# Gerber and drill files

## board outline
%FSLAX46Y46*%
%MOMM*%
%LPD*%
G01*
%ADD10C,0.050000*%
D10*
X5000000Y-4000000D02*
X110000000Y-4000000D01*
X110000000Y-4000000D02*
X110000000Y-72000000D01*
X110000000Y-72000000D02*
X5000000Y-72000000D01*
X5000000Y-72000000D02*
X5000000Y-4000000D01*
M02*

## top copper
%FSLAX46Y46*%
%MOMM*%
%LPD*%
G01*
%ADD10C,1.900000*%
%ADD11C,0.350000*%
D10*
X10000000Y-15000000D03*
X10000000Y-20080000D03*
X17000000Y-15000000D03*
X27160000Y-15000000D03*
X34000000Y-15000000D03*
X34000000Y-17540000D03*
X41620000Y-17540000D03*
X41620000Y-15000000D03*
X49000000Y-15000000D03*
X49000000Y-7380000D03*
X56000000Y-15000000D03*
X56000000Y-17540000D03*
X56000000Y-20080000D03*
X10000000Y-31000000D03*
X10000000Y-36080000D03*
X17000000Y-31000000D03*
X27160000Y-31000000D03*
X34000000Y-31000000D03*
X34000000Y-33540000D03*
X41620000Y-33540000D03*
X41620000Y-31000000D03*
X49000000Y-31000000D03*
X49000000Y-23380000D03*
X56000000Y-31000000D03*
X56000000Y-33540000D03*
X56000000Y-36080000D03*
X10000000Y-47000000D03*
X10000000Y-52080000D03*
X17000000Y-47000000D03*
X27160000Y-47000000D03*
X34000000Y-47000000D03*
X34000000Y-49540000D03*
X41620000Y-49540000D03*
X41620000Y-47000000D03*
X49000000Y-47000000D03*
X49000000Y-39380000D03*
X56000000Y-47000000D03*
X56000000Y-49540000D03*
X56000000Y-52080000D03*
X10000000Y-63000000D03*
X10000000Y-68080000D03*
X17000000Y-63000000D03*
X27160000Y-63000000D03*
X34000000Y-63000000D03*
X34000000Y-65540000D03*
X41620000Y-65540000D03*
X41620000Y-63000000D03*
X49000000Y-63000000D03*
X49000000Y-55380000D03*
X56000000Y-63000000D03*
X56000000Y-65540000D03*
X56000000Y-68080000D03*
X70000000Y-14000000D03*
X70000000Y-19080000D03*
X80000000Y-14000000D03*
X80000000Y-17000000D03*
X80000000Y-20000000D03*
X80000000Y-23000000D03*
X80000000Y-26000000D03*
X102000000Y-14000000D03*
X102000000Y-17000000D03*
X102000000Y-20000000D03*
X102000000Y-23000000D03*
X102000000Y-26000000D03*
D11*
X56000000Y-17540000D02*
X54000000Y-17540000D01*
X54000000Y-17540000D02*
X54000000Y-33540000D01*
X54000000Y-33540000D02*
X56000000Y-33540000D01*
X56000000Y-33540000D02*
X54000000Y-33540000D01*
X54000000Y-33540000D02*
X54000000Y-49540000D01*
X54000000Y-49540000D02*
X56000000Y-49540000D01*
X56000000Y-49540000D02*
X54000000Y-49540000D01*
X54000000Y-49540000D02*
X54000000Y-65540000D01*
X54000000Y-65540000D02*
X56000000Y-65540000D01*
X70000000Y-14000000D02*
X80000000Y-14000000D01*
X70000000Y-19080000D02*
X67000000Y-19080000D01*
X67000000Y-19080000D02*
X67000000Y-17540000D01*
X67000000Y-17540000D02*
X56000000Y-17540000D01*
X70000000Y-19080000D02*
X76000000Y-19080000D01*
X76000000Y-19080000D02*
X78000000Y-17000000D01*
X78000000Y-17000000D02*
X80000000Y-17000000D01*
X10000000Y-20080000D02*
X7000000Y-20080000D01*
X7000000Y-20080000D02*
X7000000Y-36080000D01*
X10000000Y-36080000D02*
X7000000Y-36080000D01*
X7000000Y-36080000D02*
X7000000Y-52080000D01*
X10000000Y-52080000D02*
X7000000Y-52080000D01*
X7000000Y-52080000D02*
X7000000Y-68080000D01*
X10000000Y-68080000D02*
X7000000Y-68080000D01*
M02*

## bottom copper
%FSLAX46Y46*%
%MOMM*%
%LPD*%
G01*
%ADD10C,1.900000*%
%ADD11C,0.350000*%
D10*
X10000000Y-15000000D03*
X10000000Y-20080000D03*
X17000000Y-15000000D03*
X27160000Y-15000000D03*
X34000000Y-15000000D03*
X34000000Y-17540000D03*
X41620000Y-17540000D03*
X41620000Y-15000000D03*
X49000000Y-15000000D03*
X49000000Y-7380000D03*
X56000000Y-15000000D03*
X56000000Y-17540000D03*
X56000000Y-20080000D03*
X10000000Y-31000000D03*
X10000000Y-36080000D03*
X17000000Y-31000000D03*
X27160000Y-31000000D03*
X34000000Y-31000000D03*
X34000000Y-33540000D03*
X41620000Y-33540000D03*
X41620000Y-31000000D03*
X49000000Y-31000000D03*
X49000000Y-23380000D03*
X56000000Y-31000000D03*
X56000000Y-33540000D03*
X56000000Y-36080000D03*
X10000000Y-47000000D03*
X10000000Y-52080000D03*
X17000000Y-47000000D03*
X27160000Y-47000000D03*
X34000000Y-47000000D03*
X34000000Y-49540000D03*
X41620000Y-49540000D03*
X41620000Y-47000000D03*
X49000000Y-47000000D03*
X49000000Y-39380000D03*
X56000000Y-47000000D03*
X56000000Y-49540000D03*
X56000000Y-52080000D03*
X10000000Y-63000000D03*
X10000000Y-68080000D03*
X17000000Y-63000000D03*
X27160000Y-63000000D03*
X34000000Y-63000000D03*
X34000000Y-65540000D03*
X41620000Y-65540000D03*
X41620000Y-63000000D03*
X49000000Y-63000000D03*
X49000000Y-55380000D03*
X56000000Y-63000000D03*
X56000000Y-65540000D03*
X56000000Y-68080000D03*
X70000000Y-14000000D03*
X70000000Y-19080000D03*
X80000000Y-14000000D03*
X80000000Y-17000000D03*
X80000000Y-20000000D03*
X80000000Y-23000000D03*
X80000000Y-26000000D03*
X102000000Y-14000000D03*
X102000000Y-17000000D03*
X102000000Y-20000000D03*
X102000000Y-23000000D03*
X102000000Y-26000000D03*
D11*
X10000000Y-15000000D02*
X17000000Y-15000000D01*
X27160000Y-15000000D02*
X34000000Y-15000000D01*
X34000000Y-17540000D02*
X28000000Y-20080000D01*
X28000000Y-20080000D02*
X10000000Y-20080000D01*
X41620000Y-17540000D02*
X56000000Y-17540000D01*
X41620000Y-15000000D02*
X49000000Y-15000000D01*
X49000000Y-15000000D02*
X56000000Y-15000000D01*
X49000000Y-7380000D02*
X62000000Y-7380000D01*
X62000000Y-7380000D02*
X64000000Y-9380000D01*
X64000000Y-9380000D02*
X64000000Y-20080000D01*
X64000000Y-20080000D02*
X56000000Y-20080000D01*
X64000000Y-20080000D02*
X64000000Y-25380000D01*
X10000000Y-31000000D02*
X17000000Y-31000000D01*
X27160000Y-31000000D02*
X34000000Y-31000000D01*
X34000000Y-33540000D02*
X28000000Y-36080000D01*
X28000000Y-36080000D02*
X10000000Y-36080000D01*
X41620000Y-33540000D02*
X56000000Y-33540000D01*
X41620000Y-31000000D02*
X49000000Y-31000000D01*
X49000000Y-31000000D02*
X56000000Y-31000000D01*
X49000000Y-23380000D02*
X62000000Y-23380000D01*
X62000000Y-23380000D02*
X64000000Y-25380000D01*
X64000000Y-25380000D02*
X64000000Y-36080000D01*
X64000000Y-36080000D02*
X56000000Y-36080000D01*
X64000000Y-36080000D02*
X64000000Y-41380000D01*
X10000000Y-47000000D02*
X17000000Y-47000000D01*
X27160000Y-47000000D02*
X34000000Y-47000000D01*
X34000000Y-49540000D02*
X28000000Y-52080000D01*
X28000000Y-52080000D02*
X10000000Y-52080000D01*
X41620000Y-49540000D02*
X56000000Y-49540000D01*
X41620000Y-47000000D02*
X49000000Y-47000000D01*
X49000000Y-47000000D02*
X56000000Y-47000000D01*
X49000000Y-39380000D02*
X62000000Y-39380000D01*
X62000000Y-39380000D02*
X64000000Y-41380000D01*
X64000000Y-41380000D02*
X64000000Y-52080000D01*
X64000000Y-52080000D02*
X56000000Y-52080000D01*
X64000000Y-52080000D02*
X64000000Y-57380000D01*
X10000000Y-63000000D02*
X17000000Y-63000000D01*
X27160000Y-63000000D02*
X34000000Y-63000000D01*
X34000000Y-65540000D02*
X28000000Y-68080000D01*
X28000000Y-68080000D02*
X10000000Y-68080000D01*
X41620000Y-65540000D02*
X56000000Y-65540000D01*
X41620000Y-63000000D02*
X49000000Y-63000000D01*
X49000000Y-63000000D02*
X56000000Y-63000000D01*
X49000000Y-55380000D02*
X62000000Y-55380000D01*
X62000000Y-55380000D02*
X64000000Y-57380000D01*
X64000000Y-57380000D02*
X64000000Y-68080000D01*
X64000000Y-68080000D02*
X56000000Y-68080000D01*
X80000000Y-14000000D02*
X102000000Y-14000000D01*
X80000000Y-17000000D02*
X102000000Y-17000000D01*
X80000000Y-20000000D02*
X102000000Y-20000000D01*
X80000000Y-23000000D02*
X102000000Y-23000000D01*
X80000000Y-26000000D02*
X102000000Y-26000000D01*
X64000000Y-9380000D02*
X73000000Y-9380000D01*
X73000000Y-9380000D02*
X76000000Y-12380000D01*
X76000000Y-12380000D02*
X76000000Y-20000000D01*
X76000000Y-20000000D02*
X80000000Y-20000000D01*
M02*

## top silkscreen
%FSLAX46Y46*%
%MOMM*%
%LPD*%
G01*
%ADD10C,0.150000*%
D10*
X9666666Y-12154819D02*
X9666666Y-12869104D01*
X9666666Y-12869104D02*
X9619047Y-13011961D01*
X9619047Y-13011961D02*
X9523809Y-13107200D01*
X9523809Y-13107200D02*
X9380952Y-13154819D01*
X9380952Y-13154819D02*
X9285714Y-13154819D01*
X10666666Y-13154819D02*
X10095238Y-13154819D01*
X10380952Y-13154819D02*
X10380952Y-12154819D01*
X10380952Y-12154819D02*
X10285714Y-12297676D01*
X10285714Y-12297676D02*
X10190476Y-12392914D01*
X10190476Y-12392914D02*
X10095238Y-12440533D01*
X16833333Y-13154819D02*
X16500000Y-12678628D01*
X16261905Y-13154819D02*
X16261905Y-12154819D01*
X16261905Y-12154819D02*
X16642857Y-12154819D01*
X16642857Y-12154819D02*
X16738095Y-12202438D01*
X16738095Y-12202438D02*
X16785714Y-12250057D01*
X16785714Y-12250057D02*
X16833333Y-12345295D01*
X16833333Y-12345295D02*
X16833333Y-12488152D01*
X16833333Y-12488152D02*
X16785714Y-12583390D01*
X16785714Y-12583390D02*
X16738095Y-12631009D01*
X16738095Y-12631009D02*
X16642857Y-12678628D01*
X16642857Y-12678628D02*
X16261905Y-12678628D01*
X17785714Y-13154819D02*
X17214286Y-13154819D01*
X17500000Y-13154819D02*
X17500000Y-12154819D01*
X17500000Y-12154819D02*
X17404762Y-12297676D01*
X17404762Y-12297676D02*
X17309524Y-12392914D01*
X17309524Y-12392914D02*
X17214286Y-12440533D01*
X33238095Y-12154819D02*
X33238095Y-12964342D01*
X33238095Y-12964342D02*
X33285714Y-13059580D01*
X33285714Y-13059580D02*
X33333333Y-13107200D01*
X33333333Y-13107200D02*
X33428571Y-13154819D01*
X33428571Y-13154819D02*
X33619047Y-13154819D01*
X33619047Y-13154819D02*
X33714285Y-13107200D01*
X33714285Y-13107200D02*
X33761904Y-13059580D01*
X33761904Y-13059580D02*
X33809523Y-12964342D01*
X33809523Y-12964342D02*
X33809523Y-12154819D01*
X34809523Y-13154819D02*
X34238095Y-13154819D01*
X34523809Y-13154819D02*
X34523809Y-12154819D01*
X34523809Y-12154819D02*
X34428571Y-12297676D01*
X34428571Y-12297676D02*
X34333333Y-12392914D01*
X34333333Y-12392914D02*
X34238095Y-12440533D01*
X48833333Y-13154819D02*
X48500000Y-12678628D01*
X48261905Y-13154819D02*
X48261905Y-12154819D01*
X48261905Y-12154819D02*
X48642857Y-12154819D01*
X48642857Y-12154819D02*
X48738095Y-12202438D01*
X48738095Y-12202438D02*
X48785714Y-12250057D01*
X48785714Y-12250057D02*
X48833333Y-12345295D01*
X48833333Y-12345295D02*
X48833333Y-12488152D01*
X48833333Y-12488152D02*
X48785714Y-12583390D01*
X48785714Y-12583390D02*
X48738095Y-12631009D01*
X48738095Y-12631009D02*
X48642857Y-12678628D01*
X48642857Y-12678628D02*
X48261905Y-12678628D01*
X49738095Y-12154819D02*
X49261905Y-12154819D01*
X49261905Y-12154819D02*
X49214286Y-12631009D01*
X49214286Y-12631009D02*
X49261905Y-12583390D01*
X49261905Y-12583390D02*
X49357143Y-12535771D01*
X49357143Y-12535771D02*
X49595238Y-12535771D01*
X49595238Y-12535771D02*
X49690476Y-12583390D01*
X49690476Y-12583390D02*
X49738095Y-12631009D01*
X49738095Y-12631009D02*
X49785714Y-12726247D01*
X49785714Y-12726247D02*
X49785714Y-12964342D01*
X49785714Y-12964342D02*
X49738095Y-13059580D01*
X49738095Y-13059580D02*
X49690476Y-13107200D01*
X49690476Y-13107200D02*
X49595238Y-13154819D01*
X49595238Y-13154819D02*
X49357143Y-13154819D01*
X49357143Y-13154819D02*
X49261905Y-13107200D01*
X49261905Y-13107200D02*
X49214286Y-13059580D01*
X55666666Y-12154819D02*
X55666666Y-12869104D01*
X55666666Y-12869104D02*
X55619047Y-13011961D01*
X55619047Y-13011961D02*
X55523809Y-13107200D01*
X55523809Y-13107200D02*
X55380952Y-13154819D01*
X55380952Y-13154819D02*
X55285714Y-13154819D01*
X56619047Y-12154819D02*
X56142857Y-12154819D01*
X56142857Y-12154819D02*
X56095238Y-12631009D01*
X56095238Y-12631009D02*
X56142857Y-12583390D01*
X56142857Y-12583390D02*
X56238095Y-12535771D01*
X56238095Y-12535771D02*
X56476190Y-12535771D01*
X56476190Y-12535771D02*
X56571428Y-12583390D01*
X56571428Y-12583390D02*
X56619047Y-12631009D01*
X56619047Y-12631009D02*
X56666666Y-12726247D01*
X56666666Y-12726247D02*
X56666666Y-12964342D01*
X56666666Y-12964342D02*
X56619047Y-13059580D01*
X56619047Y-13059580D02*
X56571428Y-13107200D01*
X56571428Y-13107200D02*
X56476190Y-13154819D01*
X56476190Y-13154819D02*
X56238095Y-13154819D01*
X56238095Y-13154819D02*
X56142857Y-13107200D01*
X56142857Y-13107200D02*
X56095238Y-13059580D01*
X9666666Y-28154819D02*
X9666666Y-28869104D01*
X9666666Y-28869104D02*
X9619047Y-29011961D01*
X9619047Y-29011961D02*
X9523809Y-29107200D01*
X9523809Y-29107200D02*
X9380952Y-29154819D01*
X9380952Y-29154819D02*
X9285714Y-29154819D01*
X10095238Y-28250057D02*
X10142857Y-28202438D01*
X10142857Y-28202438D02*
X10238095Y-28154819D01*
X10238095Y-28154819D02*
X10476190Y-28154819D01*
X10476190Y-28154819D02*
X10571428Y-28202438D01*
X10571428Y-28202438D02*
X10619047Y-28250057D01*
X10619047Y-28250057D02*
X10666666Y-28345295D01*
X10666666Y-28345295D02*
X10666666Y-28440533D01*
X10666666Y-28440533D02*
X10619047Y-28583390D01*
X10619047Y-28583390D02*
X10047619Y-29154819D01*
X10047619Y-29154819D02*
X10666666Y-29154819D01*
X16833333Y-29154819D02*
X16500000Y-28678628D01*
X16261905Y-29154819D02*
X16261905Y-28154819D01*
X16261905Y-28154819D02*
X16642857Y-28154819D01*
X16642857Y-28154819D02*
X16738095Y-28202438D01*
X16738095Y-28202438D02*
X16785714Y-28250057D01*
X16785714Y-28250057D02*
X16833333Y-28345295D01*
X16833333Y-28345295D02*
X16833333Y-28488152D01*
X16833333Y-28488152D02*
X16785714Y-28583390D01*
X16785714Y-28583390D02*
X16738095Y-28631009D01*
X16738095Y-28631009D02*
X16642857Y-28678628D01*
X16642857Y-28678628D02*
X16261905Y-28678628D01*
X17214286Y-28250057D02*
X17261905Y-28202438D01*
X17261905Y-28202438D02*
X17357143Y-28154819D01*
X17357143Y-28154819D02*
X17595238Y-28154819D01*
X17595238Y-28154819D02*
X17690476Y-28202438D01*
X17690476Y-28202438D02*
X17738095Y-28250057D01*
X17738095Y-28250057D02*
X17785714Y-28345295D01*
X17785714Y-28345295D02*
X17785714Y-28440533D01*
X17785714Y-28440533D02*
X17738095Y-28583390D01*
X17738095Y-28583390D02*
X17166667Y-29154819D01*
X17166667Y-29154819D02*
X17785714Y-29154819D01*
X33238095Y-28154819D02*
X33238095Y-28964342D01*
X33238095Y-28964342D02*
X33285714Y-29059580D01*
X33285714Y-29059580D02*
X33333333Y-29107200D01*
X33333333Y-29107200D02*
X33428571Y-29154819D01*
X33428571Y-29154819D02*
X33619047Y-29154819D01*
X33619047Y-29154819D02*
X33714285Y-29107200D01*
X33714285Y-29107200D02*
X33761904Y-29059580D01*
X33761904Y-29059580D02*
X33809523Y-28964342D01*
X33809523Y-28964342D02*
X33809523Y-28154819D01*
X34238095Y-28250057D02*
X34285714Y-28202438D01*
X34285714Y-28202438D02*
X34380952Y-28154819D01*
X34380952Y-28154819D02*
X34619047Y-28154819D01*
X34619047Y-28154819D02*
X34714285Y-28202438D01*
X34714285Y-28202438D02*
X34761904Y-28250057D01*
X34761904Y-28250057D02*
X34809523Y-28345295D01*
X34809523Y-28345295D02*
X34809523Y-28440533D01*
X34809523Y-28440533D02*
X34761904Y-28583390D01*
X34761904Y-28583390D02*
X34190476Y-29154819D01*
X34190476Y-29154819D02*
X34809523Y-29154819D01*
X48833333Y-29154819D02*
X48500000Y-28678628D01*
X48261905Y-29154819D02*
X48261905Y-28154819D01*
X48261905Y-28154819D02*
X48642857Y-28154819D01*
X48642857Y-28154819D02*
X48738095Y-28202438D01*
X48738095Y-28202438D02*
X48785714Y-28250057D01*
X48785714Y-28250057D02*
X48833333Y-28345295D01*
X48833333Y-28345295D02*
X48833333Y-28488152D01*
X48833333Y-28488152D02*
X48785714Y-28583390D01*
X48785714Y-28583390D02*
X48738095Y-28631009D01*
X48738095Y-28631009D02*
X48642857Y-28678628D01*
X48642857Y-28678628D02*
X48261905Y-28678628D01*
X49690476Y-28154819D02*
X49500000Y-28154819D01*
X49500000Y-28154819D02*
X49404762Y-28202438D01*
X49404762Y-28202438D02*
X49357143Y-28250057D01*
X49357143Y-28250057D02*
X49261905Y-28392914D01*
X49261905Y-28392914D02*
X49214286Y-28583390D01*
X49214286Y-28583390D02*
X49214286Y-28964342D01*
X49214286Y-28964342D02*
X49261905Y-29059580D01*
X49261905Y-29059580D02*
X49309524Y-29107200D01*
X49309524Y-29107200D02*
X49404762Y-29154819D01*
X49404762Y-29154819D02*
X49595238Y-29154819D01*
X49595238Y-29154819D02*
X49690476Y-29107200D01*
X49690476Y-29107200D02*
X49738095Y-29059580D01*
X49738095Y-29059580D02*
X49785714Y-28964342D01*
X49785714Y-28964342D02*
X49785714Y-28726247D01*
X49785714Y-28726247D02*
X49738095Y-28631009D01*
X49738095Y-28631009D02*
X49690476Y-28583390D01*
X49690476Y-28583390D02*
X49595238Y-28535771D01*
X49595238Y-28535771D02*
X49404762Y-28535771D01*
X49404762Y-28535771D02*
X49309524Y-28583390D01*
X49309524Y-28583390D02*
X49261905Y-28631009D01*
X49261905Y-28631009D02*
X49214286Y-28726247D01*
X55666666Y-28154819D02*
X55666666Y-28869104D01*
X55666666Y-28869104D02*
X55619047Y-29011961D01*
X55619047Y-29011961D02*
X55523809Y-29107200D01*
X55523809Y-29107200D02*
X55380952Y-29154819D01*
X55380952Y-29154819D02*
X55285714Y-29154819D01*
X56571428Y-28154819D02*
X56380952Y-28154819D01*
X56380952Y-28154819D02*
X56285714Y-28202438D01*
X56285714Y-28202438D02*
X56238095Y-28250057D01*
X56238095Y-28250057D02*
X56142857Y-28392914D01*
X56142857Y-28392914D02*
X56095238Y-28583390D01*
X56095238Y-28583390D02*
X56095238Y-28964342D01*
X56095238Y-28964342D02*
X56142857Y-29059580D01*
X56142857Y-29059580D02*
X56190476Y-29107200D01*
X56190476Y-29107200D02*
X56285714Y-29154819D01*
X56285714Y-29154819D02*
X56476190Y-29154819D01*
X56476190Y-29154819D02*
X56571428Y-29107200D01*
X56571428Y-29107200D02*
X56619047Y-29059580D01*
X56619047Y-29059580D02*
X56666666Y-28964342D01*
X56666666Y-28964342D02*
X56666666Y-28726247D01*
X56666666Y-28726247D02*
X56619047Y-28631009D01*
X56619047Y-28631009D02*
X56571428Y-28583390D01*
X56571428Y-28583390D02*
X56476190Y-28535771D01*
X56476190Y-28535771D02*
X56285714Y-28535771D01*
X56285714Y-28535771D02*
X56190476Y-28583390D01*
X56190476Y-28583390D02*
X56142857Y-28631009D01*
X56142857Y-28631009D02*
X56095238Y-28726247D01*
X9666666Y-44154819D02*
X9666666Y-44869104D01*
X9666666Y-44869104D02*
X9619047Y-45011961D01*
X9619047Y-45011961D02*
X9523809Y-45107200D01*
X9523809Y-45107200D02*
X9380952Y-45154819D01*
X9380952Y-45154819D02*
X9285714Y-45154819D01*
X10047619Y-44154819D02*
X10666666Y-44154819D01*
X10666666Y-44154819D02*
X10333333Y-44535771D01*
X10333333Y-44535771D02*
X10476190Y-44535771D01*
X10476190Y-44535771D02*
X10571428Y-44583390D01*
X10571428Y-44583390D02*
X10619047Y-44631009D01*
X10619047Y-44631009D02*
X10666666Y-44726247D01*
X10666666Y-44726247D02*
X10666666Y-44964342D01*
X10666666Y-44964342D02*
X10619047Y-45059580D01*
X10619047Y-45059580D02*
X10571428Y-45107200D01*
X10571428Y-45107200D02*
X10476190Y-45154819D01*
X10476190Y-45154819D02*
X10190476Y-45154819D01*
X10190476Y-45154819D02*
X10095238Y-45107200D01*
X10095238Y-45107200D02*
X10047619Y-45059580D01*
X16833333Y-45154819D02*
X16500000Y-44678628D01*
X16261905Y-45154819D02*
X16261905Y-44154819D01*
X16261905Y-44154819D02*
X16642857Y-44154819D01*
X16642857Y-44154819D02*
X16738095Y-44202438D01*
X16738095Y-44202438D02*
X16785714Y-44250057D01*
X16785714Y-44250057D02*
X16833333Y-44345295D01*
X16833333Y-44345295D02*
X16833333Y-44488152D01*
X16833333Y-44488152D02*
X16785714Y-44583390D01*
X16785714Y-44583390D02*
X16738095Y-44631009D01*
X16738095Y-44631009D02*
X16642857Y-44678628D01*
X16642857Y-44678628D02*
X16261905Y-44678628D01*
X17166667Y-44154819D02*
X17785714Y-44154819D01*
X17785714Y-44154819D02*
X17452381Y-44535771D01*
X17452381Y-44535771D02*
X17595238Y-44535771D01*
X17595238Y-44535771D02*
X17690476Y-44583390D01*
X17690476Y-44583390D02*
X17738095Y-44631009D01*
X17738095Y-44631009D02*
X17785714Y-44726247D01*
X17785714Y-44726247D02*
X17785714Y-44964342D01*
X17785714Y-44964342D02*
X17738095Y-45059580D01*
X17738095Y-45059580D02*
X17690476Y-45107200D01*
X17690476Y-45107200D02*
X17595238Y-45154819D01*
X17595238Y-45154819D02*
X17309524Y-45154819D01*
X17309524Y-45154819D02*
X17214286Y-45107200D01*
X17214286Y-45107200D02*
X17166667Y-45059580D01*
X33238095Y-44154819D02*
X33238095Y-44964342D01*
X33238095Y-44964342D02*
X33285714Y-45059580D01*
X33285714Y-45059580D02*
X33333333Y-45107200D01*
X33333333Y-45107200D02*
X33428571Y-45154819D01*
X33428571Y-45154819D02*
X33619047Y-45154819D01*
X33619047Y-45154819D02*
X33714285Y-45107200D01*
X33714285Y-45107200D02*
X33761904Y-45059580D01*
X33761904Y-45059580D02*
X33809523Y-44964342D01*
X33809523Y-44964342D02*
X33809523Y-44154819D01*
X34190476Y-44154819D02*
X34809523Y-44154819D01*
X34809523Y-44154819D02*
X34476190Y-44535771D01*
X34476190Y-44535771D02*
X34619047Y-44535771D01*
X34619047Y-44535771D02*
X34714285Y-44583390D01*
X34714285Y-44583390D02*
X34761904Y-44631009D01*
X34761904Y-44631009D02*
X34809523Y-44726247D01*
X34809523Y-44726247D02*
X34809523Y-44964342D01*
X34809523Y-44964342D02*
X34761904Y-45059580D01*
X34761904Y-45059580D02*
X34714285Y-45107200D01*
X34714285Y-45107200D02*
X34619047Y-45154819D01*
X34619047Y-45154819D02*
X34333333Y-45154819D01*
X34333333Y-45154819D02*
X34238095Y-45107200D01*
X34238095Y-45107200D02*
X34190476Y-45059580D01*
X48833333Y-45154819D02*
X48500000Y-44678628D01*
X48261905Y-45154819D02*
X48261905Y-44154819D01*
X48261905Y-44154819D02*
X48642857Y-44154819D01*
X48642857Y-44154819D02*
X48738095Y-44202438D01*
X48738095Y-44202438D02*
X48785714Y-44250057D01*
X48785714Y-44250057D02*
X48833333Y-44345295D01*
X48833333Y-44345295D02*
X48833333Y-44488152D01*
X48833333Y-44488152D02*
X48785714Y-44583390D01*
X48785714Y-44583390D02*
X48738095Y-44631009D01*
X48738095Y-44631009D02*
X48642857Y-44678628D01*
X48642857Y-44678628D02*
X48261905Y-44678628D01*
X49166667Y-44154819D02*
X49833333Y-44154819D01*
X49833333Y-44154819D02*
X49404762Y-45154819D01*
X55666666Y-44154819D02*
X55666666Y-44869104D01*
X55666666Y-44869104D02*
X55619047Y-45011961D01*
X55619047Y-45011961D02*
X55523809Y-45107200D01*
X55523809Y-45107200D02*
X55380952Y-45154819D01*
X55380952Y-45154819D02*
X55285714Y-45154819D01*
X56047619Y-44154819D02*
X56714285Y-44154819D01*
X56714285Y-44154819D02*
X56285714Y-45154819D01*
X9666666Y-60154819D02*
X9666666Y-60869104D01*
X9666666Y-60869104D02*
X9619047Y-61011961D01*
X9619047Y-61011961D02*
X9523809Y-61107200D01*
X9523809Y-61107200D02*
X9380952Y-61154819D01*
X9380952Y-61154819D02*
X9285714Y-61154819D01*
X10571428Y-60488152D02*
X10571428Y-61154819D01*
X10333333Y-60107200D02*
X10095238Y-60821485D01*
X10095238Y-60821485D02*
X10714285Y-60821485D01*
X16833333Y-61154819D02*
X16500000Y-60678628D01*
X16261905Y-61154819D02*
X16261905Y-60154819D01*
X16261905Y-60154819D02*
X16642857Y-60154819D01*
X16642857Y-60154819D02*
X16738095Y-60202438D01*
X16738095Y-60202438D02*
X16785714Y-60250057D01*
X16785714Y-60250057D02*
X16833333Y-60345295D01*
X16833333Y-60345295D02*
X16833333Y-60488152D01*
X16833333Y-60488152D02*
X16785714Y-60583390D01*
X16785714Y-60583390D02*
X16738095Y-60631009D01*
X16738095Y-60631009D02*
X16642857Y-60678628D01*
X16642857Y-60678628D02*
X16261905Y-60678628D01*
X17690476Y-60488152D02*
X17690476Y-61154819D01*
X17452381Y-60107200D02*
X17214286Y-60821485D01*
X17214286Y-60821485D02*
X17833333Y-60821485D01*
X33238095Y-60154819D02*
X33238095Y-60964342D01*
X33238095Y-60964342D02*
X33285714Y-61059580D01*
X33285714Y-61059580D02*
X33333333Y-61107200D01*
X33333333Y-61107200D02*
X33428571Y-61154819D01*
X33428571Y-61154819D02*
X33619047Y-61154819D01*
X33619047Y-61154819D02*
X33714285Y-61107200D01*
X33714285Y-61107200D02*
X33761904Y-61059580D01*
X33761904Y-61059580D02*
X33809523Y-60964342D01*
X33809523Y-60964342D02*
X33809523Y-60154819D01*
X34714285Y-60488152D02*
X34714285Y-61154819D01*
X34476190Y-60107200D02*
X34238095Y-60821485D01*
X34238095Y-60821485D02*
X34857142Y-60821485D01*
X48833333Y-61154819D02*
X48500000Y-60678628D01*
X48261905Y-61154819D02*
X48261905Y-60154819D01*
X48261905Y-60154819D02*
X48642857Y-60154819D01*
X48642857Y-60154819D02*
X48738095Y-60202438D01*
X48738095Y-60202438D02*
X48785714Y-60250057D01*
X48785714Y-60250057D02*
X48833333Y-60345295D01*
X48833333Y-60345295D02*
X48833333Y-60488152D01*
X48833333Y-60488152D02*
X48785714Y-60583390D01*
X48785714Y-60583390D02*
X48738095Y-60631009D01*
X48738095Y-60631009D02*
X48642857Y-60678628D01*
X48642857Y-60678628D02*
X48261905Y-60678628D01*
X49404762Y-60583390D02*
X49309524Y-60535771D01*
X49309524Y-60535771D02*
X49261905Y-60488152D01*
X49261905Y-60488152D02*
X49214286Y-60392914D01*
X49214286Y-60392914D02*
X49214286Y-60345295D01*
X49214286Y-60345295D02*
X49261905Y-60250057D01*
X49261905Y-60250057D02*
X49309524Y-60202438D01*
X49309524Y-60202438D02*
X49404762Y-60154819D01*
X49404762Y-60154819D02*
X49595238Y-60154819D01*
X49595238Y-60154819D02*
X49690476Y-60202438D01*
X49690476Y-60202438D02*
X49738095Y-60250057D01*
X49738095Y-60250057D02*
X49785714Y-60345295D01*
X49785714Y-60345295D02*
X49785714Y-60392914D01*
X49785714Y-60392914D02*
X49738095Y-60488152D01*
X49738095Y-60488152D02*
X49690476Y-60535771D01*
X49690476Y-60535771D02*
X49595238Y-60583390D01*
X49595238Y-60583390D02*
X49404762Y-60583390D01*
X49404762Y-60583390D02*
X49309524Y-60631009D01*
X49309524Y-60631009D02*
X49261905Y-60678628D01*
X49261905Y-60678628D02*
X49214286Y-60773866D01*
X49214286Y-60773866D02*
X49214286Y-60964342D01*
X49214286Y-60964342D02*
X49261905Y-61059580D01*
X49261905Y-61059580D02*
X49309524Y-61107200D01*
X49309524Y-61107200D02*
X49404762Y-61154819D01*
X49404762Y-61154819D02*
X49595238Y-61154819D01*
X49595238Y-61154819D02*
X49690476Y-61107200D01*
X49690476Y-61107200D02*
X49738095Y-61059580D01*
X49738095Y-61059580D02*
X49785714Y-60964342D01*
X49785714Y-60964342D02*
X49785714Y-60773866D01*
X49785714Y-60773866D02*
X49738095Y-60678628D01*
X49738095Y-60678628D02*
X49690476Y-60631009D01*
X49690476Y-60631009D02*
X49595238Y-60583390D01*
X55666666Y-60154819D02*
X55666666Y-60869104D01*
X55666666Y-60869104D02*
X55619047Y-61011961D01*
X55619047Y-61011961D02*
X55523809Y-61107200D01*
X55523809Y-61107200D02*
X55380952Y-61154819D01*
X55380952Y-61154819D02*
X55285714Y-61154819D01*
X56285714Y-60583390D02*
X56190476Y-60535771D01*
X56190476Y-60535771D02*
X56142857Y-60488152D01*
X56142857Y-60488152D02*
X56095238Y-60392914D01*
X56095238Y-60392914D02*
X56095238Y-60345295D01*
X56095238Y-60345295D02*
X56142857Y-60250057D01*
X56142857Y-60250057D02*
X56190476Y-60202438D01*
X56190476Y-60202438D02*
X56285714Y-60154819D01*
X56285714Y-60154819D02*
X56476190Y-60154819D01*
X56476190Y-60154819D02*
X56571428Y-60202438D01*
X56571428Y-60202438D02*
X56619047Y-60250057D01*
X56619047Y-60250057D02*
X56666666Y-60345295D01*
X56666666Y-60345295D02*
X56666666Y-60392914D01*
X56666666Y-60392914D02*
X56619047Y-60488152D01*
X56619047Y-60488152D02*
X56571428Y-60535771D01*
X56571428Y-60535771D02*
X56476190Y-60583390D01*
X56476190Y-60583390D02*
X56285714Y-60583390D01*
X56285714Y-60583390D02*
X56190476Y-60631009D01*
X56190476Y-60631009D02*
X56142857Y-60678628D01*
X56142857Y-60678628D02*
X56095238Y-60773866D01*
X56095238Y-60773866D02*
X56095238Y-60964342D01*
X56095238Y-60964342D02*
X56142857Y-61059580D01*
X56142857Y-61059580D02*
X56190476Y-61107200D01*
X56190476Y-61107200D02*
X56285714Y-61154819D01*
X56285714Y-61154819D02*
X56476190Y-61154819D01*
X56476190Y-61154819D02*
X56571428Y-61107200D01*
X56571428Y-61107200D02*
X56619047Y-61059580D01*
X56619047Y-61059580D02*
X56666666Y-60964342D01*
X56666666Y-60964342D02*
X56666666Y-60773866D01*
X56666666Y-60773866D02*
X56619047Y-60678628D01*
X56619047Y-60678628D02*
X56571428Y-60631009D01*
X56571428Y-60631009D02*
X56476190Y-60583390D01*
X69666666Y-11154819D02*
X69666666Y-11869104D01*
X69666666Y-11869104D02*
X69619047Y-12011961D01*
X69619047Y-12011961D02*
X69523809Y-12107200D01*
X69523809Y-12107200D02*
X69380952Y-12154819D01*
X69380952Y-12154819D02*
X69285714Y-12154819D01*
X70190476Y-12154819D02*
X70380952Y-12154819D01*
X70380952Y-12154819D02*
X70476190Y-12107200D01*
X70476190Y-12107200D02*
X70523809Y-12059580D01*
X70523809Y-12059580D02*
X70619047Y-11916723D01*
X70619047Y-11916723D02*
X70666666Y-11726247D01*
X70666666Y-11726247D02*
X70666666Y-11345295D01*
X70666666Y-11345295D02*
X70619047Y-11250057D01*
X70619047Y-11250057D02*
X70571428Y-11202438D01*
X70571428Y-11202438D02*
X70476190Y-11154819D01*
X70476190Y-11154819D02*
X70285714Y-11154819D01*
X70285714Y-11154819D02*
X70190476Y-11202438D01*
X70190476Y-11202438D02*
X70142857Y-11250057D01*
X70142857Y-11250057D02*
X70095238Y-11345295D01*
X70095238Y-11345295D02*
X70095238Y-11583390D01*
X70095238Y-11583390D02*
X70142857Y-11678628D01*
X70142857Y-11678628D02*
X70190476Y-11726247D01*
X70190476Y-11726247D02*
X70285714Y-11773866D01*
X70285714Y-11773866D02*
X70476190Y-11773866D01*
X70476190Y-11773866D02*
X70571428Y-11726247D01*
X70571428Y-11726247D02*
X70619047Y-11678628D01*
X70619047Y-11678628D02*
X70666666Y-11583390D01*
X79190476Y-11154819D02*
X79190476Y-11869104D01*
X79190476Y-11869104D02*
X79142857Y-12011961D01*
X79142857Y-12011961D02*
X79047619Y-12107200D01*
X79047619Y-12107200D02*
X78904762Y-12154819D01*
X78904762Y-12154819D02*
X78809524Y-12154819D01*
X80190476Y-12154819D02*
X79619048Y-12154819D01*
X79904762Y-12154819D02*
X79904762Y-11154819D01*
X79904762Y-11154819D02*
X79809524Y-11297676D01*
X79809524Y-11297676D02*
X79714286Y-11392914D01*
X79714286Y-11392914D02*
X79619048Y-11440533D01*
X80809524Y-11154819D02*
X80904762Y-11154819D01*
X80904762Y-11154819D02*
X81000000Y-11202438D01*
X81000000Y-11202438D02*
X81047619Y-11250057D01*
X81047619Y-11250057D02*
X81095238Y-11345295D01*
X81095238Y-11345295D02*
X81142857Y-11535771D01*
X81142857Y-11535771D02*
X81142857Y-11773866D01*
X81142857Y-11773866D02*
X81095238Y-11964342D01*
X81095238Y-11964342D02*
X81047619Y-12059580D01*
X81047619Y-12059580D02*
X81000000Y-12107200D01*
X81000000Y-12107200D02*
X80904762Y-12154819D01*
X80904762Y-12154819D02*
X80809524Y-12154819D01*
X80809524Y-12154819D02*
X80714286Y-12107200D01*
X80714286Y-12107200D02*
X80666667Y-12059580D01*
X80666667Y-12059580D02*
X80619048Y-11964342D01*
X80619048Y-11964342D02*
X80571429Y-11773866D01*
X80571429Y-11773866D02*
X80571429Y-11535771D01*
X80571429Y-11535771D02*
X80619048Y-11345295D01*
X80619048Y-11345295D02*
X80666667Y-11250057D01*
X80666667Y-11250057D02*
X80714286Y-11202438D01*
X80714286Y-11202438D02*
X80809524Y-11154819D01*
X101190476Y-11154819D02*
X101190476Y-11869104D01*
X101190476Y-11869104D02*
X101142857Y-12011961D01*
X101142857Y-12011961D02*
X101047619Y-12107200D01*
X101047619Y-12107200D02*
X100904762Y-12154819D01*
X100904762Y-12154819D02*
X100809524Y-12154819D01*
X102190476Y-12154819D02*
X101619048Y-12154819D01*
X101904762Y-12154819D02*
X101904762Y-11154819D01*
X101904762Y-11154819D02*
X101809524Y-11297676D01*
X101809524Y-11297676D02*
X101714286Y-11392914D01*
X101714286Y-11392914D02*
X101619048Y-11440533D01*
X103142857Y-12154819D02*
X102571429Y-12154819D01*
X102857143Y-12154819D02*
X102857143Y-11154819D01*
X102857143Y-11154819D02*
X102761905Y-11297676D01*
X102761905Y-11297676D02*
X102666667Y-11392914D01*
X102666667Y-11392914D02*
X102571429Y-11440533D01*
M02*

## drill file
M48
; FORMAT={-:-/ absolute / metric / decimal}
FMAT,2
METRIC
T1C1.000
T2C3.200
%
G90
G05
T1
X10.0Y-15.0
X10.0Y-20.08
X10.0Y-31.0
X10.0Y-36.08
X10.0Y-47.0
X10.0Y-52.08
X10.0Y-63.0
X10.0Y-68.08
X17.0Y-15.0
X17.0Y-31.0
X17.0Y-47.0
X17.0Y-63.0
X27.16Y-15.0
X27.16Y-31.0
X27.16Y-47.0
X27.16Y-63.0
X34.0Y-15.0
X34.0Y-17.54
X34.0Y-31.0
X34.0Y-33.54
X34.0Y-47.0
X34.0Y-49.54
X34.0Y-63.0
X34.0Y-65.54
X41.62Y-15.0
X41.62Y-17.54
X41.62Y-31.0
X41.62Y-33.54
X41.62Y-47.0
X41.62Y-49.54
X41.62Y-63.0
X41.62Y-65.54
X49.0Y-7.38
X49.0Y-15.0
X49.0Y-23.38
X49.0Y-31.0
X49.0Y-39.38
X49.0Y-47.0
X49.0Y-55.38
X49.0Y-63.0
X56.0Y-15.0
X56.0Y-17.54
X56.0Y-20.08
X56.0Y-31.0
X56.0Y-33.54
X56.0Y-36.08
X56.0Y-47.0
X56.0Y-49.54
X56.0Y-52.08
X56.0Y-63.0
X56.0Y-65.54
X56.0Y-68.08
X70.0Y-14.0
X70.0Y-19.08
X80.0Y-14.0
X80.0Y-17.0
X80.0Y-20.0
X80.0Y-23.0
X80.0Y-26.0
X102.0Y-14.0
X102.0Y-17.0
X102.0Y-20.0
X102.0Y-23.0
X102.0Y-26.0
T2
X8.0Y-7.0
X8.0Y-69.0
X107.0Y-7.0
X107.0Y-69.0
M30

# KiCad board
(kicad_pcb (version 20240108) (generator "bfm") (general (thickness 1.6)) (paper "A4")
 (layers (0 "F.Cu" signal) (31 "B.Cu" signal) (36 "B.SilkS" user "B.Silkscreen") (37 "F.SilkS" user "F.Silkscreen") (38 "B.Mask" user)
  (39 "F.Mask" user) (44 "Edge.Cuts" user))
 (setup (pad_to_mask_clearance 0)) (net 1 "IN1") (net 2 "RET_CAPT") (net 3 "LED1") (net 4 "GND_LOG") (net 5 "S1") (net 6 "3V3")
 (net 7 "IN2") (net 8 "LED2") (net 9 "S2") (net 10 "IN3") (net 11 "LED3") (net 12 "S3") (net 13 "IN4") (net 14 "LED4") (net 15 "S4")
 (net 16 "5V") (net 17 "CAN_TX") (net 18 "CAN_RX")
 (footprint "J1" (layer "F.Cu") (at 10 15)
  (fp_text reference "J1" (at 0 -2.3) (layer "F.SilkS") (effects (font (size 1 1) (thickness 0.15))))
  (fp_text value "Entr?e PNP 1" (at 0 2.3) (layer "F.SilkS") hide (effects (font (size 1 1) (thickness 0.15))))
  (pad "1" thru_hole circle (at 0.0000 0.0000) (size 1.9 1.9) (drill 1) (layers "*.Cu" "*.Mask") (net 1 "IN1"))
  (pad "2" thru_hole circle (at 0.0000 5.0800) (size 1.9 1.9) (drill 1) (layers "*.Cu" "*.Mask") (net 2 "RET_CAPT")))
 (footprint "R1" (layer "F.Cu") (at 17 15)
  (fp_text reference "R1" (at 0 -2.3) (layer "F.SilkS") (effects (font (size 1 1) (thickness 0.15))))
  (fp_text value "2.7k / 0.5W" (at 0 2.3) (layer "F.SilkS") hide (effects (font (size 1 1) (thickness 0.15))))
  (pad "1" thru_hole circle (at 0.0000 0.0000) (size 1.9 1.9) (drill 1) (layers "*.Cu" "*.Mask") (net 1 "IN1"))
  (pad "2" thru_hole circle (at 10.1600 0.0000) (size 1.9 1.9) (drill 1) (layers "*.Cu" "*.Mask") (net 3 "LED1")))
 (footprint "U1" (layer "F.Cu") (at 34 15)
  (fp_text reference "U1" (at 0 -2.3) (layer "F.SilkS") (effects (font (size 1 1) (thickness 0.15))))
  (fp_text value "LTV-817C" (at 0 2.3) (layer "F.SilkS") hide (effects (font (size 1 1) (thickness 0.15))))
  (pad "1" thru_hole circle (at 0.0000 0.0000) (size 1.9 1.9) (drill 1) (layers "*.Cu" "*.Mask") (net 3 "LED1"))
  (pad "2" thru_hole circle (at 0.0000 2.5400) (size 1.9 1.9) (drill 1) (layers "*.Cu" "*.Mask") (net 2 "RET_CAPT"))
  (pad "3" thru_hole circle (at 7.6200 2.5400) (size 1.9 1.9) (drill 1) (layers "*.Cu" "*.Mask") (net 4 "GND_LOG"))
  (pad "4" thru_hole circle (at 7.6200 0.0000) (size 1.9 1.9) (drill 1) (layers "*.Cu" "*.Mask") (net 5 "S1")))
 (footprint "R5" (layer "F.Cu") (at 49 15)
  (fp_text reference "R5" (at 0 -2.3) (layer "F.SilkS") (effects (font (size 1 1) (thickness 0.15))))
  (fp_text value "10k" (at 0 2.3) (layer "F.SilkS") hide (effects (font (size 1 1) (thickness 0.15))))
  (pad "1" thru_hole circle (at 0.0000 0.0000) (size 1.9 1.9) (drill 1) (layers "*.Cu" "*.Mask") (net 5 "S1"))
  (pad "2" thru_hole circle (at 0.0000 -7.6200) (size 1.9 1.9) (drill 1) (layers "*.Cu" "*.Mask") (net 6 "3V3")))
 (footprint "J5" (layer "F.Cu") (at 56 15)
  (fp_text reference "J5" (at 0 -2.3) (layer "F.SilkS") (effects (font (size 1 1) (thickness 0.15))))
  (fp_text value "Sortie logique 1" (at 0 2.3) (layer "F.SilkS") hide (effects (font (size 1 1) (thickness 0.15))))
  (pad "1" thru_hole circle (at 0.0000 0.0000) (size 1.9 1.9) (drill 1) (layers "*.Cu" "*.Mask") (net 5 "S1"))
  (pad "2" thru_hole circle (at 0.0000 2.5400) (size 1.9 1.9) (drill 1) (layers "*.Cu" "*.Mask") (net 4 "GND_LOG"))
  (pad "3" thru_hole circle (at 0.0000 5.0800) (size 1.9 1.9) (drill 1) (layers "*.Cu" "*.Mask") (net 6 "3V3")))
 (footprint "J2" (layer "F.Cu") (at 10 31)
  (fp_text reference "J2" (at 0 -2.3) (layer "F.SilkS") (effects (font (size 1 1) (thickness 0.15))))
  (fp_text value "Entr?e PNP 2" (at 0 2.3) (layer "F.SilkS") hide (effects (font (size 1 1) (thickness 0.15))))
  (pad "1" thru_hole circle (at 0.0000 0.0000) (size 1.9 1.9) (drill 1) (layers "*.Cu" "*.Mask") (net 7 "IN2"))
  (pad "2" thru_hole circle (at 0.0000 5.0800) (size 1.9 1.9) (drill 1) (layers "*.Cu" "*.Mask") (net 2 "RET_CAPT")))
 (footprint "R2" (layer "F.Cu") (at 17 31)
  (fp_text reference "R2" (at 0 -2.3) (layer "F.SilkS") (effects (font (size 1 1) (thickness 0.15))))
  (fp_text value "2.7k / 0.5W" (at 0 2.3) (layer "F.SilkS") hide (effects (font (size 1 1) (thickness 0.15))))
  (pad "1" thru_hole circle (at 0.0000 0.0000) (size 1.9 1.9) (drill 1) (layers "*.Cu" "*.Mask") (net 7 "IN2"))
  (pad "2" thru_hole circle (at 10.1600 0.0000) (size 1.9 1.9) (drill 1) (layers "*.Cu" "*.Mask") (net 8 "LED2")))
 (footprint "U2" (layer "F.Cu") (at 34 31)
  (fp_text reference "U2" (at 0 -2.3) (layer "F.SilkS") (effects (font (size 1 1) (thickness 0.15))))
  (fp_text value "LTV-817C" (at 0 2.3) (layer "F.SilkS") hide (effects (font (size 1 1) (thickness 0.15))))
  (pad "1" thru_hole circle (at 0.0000 0.0000) (size 1.9 1.9) (drill 1) (layers "*.Cu" "*.Mask") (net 8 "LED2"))
  (pad "2" thru_hole circle (at 0.0000 2.5400) (size 1.9 1.9) (drill 1) (layers "*.Cu" "*.Mask") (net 2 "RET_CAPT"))
  (pad "3" thru_hole circle (at 7.6200 2.5400) (size 1.9 1.9) (drill 1) (layers "*.Cu" "*.Mask") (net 4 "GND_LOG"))
  (pad "4" thru_hole circle (at 7.6200 0.0000) (size 1.9 1.9) (drill 1) (layers "*.Cu" "*.Mask") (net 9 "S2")))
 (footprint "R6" (layer "F.Cu") (at 49 31)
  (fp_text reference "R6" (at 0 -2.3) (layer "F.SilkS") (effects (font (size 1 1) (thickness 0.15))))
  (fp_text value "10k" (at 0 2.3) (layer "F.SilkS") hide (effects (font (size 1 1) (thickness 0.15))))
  (pad "1" thru_hole circle (at 0.0000 0.0000) (size 1.9 1.9) (drill 1) (layers "*.Cu" "*.Mask") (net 9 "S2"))
  (pad "2" thru_hole circle (at 0.0000 -7.6200) (size 1.9 1.9) (drill 1) (layers "*.Cu" "*.Mask") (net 6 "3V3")))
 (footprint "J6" (layer "F.Cu") (at 56 31)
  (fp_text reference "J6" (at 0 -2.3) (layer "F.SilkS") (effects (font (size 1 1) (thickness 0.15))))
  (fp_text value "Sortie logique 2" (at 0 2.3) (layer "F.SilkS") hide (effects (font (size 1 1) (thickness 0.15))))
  (pad "1" thru_hole circle (at 0.0000 0.0000) (size 1.9 1.9) (drill 1) (layers "*.Cu" "*.Mask") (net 9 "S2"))
  (pad "2" thru_hole circle (at 0.0000 2.5400) (size 1.9 1.9) (drill 1) (layers "*.Cu" "*.Mask") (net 4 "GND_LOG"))
  (pad "3" thru_hole circle (at 0.0000 5.0800) (size 1.9 1.9) (drill 1) (layers "*.Cu" "*.Mask") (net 6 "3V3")))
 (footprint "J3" (layer "F.Cu") (at 10 47)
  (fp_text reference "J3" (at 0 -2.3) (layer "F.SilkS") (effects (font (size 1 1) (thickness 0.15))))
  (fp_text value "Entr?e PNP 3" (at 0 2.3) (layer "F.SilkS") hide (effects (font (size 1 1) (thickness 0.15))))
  (pad "1" thru_hole circle (at 0.0000 0.0000) (size 1.9 1.9) (drill 1) (layers "*.Cu" "*.Mask") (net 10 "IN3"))
  (pad "2" thru_hole circle (at 0.0000 5.0800) (size 1.9 1.9) (drill 1) (layers "*.Cu" "*.Mask") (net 2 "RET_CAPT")))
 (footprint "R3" (layer "F.Cu") (at 17 47)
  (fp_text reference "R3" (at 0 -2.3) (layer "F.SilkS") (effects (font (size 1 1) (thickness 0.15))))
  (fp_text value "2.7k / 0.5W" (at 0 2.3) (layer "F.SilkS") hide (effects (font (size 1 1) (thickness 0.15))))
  (pad "1" thru_hole circle (at 0.0000 0.0000) (size 1.9 1.9) (drill 1) (layers "*.Cu" "*.Mask") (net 10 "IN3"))
  (pad "2" thru_hole circle (at 10.1600 0.0000) (size 1.9 1.9) (drill 1) (layers "*.Cu" "*.Mask") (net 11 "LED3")))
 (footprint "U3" (layer "F.Cu") (at 34 47)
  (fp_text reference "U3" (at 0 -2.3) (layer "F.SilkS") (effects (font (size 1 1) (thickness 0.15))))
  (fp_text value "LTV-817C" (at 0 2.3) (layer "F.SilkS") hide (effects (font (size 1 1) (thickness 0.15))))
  (pad "1" thru_hole circle (at 0.0000 0.0000) (size 1.9 1.9) (drill 1) (layers "*.Cu" "*.Mask") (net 11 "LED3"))
  (pad "2" thru_hole circle (at 0.0000 2.5400) (size 1.9 1.9) (drill 1) (layers "*.Cu" "*.Mask") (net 2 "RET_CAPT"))
  (pad "3" thru_hole circle (at 7.6200 2.5400) (size 1.9 1.9) (drill 1) (layers "*.Cu" "*.Mask") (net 4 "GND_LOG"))
  (pad "4" thru_hole circle (at 7.6200 0.0000) (size 1.9 1.9) (drill 1) (layers "*.Cu" "*.Mask") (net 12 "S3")))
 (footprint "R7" (layer "F.Cu") (at 49 47)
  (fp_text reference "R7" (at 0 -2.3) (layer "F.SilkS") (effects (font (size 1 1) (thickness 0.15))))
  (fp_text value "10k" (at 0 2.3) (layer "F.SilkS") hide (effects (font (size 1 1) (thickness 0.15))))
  (pad "1" thru_hole circle (at 0.0000 0.0000) (size 1.9 1.9) (drill 1) (layers "*.Cu" "*.Mask") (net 12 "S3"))
  (pad "2" thru_hole circle (at 0.0000 -7.6200) (size 1.9 1.9) (drill 1) (layers "*.Cu" "*.Mask") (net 6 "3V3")))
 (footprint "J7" (layer "F.Cu") (at 56 47)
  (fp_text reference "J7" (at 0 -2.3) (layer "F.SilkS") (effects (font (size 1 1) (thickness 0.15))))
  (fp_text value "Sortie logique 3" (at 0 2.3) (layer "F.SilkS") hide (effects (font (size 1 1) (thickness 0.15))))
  (pad "1" thru_hole circle (at 0.0000 0.0000) (size 1.9 1.9) (drill 1) (layers "*.Cu" "*.Mask") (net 12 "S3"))
  (pad "2" thru_hole circle (at 0.0000 2.5400) (size 1.9 1.9) (drill 1) (layers "*.Cu" "*.Mask") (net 4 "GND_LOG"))
  (pad "3" thru_hole circle (at 0.0000 5.0800) (size 1.9 1.9) (drill 1) (layers "*.Cu" "*.Mask") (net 6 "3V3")))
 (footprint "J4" (layer "F.Cu") (at 10 63)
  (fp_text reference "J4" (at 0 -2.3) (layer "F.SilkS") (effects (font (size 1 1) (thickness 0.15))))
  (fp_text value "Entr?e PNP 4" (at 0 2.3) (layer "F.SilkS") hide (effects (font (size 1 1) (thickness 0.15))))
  (pad "1" thru_hole circle (at 0.0000 0.0000) (size 1.9 1.9) (drill 1) (layers "*.Cu" "*.Mask") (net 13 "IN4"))
  (pad "2" thru_hole circle (at 0.0000 5.0800) (size 1.9 1.9) (drill 1) (layers "*.Cu" "*.Mask") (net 2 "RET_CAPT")))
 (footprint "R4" (layer "F.Cu") (at 17 63)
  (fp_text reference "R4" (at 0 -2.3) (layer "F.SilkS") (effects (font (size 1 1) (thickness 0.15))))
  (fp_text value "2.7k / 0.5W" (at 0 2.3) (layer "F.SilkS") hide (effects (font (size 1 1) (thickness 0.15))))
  (pad "1" thru_hole circle (at 0.0000 0.0000) (size 1.9 1.9) (drill 1) (layers "*.Cu" "*.Mask") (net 13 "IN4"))
  (pad "2" thru_hole circle (at 10.1600 0.0000) (size 1.9 1.9) (drill 1) (layers "*.Cu" "*.Mask") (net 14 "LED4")))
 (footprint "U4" (layer "F.Cu") (at 34 63)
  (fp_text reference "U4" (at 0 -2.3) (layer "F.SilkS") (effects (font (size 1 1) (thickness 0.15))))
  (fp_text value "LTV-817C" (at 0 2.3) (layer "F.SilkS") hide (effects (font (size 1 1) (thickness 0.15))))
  (pad "1" thru_hole circle (at 0.0000 0.0000) (size 1.9 1.9) (drill 1) (layers "*.Cu" "*.Mask") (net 14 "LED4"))
  (pad "2" thru_hole circle (at 0.0000 2.5400) (size 1.9 1.9) (drill 1) (layers "*.Cu" "*.Mask") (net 2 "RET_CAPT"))
  (pad "3" thru_hole circle (at 7.6200 2.5400) (size 1.9 1.9) (drill 1) (layers "*.Cu" "*.Mask") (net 4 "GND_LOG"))
  (pad "4" thru_hole circle (at 7.6200 0.0000) (size 1.9 1.9) (drill 1) (layers "*.Cu" "*.Mask") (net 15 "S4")))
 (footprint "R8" (layer "F.Cu") (at 49 63)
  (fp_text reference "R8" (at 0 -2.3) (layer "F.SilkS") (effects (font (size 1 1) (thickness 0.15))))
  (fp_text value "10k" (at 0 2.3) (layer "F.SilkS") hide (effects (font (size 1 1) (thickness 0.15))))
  (pad "1" thru_hole circle (at 0.0000 0.0000) (size 1.9 1.9) (drill 1) (layers "*.Cu" "*.Mask") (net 15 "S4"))
  (pad "2" thru_hole circle (at 0.0000 -7.6200) (size 1.9 1.9) (drill 1) (layers "*.Cu" "*.Mask") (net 6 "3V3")))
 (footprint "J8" (layer "F.Cu") (at 56 63)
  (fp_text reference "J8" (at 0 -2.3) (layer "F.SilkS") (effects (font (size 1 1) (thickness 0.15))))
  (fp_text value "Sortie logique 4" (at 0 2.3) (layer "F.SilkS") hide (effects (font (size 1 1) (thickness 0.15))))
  (pad "1" thru_hole circle (at 0.0000 0.0000) (size 1.9 1.9) (drill 1) (layers "*.Cu" "*.Mask") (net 15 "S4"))
  (pad "2" thru_hole circle (at 0.0000 2.5400) (size 1.9 1.9) (drill 1) (layers "*.Cu" "*.Mask") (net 4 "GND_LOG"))
  (pad "3" thru_hole circle (at 0.0000 5.0800) (size 1.9 1.9) (drill 1) (layers "*.Cu" "*.Mask") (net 6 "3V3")))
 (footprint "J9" (layer "F.Cu") (at 70 14)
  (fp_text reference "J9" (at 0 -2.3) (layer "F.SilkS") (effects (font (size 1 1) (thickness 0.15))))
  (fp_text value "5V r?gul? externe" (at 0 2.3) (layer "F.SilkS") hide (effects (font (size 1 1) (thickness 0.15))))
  (pad "1" thru_hole circle (at 0.0000 0.0000) (size 1.9 1.9) (drill 1) (layers "*.Cu" "*.Mask") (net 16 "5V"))
  (pad "2" thru_hole circle (at 0.0000 5.0800) (size 1.9 1.9) (drill 1) (layers "*.Cu" "*.Mask") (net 4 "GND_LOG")))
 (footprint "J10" (layer "F.Cu") (at 80 14)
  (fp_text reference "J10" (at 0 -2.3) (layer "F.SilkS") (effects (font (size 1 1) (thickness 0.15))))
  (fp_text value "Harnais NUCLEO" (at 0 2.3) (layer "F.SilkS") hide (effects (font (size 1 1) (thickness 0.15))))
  (pad "1" thru_hole circle (at 0.0000 0.0000) (size 1.9 1.9) (drill 1) (layers "*.Cu" "*.Mask") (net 16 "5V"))
  (pad "2" thru_hole circle (at 0.0000 3.0000) (size 1.9 1.9) (drill 1) (layers "*.Cu" "*.Mask") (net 4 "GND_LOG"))
  (pad "3" thru_hole circle (at 0.0000 6.0000) (size 1.9 1.9) (drill 1) (layers "*.Cu" "*.Mask") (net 6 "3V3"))
  (pad "4" thru_hole circle (at 0.0000 9.0000) (size 1.9 1.9) (drill 1) (layers "*.Cu" "*.Mask") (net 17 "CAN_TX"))
  (pad "5" thru_hole circle (at 0.0000 12.0000) (size 1.9 1.9) (drill 1) (layers "*.Cu" "*.Mask") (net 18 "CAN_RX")))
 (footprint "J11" (layer "F.Cu") (at 102 14)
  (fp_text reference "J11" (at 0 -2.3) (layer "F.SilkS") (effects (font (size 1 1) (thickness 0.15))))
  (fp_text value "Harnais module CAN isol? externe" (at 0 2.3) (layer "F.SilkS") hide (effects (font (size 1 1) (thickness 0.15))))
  (pad "1" thru_hole circle (at 0.0000 0.0000) (size 1.9 1.9) (drill 1) (layers "*.Cu" "*.Mask") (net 16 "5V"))
  (pad "2" thru_hole circle (at 0.0000 3.0000) (size 1.9 1.9) (drill 1) (layers "*.Cu" "*.Mask") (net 4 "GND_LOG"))
  (pad "3" thru_hole circle (at 0.0000 6.0000) (size 1.9 1.9) (drill 1) (layers "*.Cu" "*.Mask") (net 6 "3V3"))
  (pad "4" thru_hole circle (at 0.0000 9.0000) (size 1.9 1.9) (drill 1) (layers "*.Cu" "*.Mask") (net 17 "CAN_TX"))
  (pad "5" thru_hole circle (at 0.0000 12.0000) (size 1.9 1.9) (drill 1) (layers "*.Cu" "*.Mask") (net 18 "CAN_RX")))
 (gr_line (start 5 4) (end 110 4) (stroke (width 0.05) (type default)) (layer "Edge.Cuts"))
 (gr_line (start 110 4) (end 110 72) (stroke (width 0.05) (type default)) (layer "Edge.Cuts"))
 (gr_line (start 110 72) (end 5 72) (stroke (width 0.05) (type default)) (layer "Edge.Cuts"))
 (gr_line (start 5 72) (end 5 4) (stroke (width 0.05) (type default)) (layer "Edge.Cuts"))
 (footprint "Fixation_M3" (layer "F.Cu") (at 8 7) (pad "" np_thru_hole circle (at 0 0) (size 3.2 3.2) (drill 3.2) (layers "*.Cu" "*.Mask")))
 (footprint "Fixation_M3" (layer "F.Cu") (at 107 7)
  (pad "" np_thru_hole circle (at 0 0) (size 3.2 3.2) (drill 3.2) (layers "*.Cu" "*.Mask")))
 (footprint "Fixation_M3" (layer "F.Cu") (at 107 69)
  (pad "" np_thru_hole circle (at 0 0) (size 3.2 3.2) (drill 3.2) (layers "*.Cu" "*.Mask")))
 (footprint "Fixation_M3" (layer "F.Cu") (at 8 69)
  (pad "" np_thru_hole circle (at 0 0) (size 3.2 3.2) (drill 3.2) (layers "*.Cu" "*.Mask")))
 (segment (start 10 15) (end 17 15) (width 0.35) (layer "B.Cu") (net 1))
 (segment (start 27.16 15) (end 34 15) (width 0.35) (layer "B.Cu") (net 3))
 (segment (start 34 17.54) (end 28 20.08) (width 0.35) (layer "B.Cu") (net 2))
 (segment (start 28 20.08) (end 10 20.08) (width 0.35) (layer "B.Cu") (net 2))
 (segment (start 41.62 17.54) (end 56 17.54) (width 0.35) (layer "B.Cu") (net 4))
 (segment (start 41.62 15) (end 49 15) (width 0.35) (layer "B.Cu") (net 5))
 (segment (start 49 15) (end 56 15) (width 0.35) (layer "B.Cu") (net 5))
 (segment (start 49 7.38) (end 62 7.38) (width 0.35) (layer "B.Cu") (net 6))
 (segment (start 62 7.38) (end 64 9.379999999999999) (width 0.35) (layer "B.Cu") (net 6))
 (segment (start 64 9.379999999999999) (end 64 20.08) (width 0.35) (layer "B.Cu") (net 6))
 (segment (start 64 20.08) (end 56 20.08) (width 0.35) (layer "B.Cu") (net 6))
 (segment (start 64 20.08) (end 64 25.380000000000003) (width 0.35) (layer "B.Cu") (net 6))
 (segment (start 56 17.54) (end 54 17.54) (width 0.35) (layer "F.Cu") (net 4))
 (segment (start 54 17.54) (end 54 33.54) (width 0.35) (layer "F.Cu") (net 4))
 (segment (start 54 33.54) (end 56 33.54) (width 0.35) (layer "F.Cu") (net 4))
 (segment (start 10 31) (end 17 31) (width 0.35) (layer "B.Cu") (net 7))
 (segment (start 27.16 31) (end 34 31) (width 0.35) (layer "B.Cu") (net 8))
 (segment (start 34 33.54) (end 28 36.08) (width 0.35) (layer "B.Cu") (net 2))
 (segment (start 28 36.08) (end 10 36.08) (width 0.35) (layer "B.Cu") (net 2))
 (segment (start 41.62 33.54) (end 56 33.54) (width 0.35) (layer "B.Cu") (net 4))
 (segment (start 41.62 31) (end 49 31) (width 0.35) (layer "B.Cu") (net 9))
 (segment (start 49 31) (end 56 31) (width 0.35) (layer "B.Cu") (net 9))
 (segment (start 49 23.38) (end 62 23.38) (width 0.35) (layer "B.Cu") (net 6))
 (segment (start 62 23.38) (end 64 25.38) (width 0.35) (layer "B.Cu") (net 6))
 (segment (start 64 25.38) (end 64 36.08) (width 0.35) (layer "B.Cu") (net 6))
 (segment (start 64 36.08) (end 56 36.08) (width 0.35) (layer "B.Cu") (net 6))
 (segment (start 64 36.08) (end 64 41.38) (width 0.35) (layer "B.Cu") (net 6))
 (segment (start 56 33.54) (end 54 33.54) (width 0.35) (layer "F.Cu") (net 4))
 (segment (start 54 33.54) (end 54 49.54) (width 0.35) (layer "F.Cu") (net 4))
 (segment (start 54 49.54) (end 56 49.54) (width 0.35) (layer "F.Cu") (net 4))
 (segment (start 10 47) (end 17 47) (width 0.35) (layer "B.Cu") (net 10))
 (segment (start 27.16 47) (end 34 47) (width 0.35) (layer "B.Cu") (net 11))
 (segment (start 34 49.54) (end 28 52.08) (width 0.35) (layer "B.Cu") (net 2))
 (segment (start 28 52.08) (end 10 52.08) (width 0.35) (layer "B.Cu") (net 2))
 (segment (start 41.62 49.54) (end 56 49.54) (width 0.35) (layer "B.Cu") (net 4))
 (segment (start 41.62 47) (end 49 47) (width 0.35) (layer "B.Cu") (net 12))
 (segment (start 49 47) (end 56 47) (width 0.35) (layer "B.Cu") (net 12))
 (segment (start 49 39.38) (end 62 39.38) (width 0.35) (layer "B.Cu") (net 6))
 (segment (start 62 39.38) (end 64 41.38) (width 0.35) (layer "B.Cu") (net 6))
 (segment (start 64 41.38) (end 64 52.08) (width 0.35) (layer "B.Cu") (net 6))
 (segment (start 64 52.08) (end 56 52.08) (width 0.35) (layer "B.Cu") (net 6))
 (segment (start 64 52.08) (end 64 57.38) (width 0.35) (layer "B.Cu") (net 6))
 (segment (start 56 49.54) (end 54 49.54) (width 0.35) (layer "F.Cu") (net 4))
 (segment (start 54 49.54) (end 54 65.53999999999999) (width 0.35) (layer "F.Cu") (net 4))
 (segment (start 54 65.53999999999999) (end 56 65.53999999999999) (width 0.35) (layer "F.Cu") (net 4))
 (segment (start 10 63) (end 17 63) (width 0.35) (layer "B.Cu") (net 13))
 (segment (start 27.16 63) (end 34 63) (width 0.35) (layer "B.Cu") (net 14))
 (segment (start 34 65.54) (end 28 68.08) (width 0.35) (layer "B.Cu") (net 2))
 (segment (start 28 68.08) (end 10 68.08) (width 0.35) (layer "B.Cu") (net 2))
 (segment (start 41.62 65.54) (end 56 65.54) (width 0.35) (layer "B.Cu") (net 4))
 (segment (start 41.62 63) (end 49 63) (width 0.35) (layer "B.Cu") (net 15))
 (segment (start 49 63) (end 56 63) (width 0.35) (layer "B.Cu") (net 15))
 (segment (start 49 55.38) (end 62 55.38) (width 0.35) (layer "B.Cu") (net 6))
 (segment (start 62 55.38) (end 64 57.38) (width 0.35) (layer "B.Cu") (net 6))
 (segment (start 64 57.38) (end 64 68.08) (width 0.35) (layer "B.Cu") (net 6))
 (segment (start 64 68.08) (end 56 68.08) (width 0.35) (layer "B.Cu") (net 6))
 (segment (start 80 14) (end 102 14) (width 0.35) (layer "B.Cu") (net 16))
 (segment (start 80 17) (end 102 17) (width 0.35) (layer "B.Cu") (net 4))
 (segment (start 80 20) (end 102 20) (width 0.35) (layer "B.Cu") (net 6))
 (segment (start 80 23) (end 102 23) (width 0.35) (layer "B.Cu") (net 17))
 (segment (start 80 26) (end 102 26) (width 0.35) (layer "B.Cu") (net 18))
 (segment (start 70 14) (end 80 14) (width 0.35) (layer "F.Cu") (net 16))
 (segment (start 70 19.08) (end 67 19.08) (width 0.35) (layer "F.Cu") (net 4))
 (segment (start 67 19.08) (end 67 17.54) (width 0.35) (layer "F.Cu") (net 4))
 (segment (start 67 17.54) (end 56 17.54) (width 0.35) (layer "F.Cu") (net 4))
 (segment (start 70 19.08) (end 76 19.08) (width 0.35) (layer "F.Cu") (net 4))
 (segment (start 76 19.08) (end 78 17) (width 0.35) (layer "F.Cu") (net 4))
 (segment (start 78 17) (end 80 17) (width 0.35) (layer "F.Cu") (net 4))
 (segment (start 64 9.38) (end 73 9.38) (width 0.35) (layer "B.Cu") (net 6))
 (segment (start 73 9.38) (end 76 12.38) (width 0.35) (layer "B.Cu") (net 6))
 (segment (start 76 12.38) (end 76 20) (width 0.35) (layer "B.Cu") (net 6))
 (segment (start 76 20) (end 80 20) (width 0.35) (layer "B.Cu") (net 6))
 (segment (start 10 20.08) (end 7 20.08) (width 0.35) (layer "F.Cu") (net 2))
 (segment (start 7 20.08) (end 7 36.08) (width 0.35) (layer "F.Cu") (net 2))
 (segment (start 10 36.08) (end 7 36.08) (width 0.35) (layer "F.Cu") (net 2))
 (segment (start 7 36.08) (end 7 52.08) (width 0.35) (layer "F.Cu") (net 2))
 (segment (start 10 52.08) (end 7 52.08) (width 0.35) (layer "F.Cu") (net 2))
 (segment (start 7 52.08) (end 7 68.08) (width 0.35) (layer "F.Cu") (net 2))
 (segment (start 10 68.08) (end 7 68.08) (width 0.35) (layer "F.Cu") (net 2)))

